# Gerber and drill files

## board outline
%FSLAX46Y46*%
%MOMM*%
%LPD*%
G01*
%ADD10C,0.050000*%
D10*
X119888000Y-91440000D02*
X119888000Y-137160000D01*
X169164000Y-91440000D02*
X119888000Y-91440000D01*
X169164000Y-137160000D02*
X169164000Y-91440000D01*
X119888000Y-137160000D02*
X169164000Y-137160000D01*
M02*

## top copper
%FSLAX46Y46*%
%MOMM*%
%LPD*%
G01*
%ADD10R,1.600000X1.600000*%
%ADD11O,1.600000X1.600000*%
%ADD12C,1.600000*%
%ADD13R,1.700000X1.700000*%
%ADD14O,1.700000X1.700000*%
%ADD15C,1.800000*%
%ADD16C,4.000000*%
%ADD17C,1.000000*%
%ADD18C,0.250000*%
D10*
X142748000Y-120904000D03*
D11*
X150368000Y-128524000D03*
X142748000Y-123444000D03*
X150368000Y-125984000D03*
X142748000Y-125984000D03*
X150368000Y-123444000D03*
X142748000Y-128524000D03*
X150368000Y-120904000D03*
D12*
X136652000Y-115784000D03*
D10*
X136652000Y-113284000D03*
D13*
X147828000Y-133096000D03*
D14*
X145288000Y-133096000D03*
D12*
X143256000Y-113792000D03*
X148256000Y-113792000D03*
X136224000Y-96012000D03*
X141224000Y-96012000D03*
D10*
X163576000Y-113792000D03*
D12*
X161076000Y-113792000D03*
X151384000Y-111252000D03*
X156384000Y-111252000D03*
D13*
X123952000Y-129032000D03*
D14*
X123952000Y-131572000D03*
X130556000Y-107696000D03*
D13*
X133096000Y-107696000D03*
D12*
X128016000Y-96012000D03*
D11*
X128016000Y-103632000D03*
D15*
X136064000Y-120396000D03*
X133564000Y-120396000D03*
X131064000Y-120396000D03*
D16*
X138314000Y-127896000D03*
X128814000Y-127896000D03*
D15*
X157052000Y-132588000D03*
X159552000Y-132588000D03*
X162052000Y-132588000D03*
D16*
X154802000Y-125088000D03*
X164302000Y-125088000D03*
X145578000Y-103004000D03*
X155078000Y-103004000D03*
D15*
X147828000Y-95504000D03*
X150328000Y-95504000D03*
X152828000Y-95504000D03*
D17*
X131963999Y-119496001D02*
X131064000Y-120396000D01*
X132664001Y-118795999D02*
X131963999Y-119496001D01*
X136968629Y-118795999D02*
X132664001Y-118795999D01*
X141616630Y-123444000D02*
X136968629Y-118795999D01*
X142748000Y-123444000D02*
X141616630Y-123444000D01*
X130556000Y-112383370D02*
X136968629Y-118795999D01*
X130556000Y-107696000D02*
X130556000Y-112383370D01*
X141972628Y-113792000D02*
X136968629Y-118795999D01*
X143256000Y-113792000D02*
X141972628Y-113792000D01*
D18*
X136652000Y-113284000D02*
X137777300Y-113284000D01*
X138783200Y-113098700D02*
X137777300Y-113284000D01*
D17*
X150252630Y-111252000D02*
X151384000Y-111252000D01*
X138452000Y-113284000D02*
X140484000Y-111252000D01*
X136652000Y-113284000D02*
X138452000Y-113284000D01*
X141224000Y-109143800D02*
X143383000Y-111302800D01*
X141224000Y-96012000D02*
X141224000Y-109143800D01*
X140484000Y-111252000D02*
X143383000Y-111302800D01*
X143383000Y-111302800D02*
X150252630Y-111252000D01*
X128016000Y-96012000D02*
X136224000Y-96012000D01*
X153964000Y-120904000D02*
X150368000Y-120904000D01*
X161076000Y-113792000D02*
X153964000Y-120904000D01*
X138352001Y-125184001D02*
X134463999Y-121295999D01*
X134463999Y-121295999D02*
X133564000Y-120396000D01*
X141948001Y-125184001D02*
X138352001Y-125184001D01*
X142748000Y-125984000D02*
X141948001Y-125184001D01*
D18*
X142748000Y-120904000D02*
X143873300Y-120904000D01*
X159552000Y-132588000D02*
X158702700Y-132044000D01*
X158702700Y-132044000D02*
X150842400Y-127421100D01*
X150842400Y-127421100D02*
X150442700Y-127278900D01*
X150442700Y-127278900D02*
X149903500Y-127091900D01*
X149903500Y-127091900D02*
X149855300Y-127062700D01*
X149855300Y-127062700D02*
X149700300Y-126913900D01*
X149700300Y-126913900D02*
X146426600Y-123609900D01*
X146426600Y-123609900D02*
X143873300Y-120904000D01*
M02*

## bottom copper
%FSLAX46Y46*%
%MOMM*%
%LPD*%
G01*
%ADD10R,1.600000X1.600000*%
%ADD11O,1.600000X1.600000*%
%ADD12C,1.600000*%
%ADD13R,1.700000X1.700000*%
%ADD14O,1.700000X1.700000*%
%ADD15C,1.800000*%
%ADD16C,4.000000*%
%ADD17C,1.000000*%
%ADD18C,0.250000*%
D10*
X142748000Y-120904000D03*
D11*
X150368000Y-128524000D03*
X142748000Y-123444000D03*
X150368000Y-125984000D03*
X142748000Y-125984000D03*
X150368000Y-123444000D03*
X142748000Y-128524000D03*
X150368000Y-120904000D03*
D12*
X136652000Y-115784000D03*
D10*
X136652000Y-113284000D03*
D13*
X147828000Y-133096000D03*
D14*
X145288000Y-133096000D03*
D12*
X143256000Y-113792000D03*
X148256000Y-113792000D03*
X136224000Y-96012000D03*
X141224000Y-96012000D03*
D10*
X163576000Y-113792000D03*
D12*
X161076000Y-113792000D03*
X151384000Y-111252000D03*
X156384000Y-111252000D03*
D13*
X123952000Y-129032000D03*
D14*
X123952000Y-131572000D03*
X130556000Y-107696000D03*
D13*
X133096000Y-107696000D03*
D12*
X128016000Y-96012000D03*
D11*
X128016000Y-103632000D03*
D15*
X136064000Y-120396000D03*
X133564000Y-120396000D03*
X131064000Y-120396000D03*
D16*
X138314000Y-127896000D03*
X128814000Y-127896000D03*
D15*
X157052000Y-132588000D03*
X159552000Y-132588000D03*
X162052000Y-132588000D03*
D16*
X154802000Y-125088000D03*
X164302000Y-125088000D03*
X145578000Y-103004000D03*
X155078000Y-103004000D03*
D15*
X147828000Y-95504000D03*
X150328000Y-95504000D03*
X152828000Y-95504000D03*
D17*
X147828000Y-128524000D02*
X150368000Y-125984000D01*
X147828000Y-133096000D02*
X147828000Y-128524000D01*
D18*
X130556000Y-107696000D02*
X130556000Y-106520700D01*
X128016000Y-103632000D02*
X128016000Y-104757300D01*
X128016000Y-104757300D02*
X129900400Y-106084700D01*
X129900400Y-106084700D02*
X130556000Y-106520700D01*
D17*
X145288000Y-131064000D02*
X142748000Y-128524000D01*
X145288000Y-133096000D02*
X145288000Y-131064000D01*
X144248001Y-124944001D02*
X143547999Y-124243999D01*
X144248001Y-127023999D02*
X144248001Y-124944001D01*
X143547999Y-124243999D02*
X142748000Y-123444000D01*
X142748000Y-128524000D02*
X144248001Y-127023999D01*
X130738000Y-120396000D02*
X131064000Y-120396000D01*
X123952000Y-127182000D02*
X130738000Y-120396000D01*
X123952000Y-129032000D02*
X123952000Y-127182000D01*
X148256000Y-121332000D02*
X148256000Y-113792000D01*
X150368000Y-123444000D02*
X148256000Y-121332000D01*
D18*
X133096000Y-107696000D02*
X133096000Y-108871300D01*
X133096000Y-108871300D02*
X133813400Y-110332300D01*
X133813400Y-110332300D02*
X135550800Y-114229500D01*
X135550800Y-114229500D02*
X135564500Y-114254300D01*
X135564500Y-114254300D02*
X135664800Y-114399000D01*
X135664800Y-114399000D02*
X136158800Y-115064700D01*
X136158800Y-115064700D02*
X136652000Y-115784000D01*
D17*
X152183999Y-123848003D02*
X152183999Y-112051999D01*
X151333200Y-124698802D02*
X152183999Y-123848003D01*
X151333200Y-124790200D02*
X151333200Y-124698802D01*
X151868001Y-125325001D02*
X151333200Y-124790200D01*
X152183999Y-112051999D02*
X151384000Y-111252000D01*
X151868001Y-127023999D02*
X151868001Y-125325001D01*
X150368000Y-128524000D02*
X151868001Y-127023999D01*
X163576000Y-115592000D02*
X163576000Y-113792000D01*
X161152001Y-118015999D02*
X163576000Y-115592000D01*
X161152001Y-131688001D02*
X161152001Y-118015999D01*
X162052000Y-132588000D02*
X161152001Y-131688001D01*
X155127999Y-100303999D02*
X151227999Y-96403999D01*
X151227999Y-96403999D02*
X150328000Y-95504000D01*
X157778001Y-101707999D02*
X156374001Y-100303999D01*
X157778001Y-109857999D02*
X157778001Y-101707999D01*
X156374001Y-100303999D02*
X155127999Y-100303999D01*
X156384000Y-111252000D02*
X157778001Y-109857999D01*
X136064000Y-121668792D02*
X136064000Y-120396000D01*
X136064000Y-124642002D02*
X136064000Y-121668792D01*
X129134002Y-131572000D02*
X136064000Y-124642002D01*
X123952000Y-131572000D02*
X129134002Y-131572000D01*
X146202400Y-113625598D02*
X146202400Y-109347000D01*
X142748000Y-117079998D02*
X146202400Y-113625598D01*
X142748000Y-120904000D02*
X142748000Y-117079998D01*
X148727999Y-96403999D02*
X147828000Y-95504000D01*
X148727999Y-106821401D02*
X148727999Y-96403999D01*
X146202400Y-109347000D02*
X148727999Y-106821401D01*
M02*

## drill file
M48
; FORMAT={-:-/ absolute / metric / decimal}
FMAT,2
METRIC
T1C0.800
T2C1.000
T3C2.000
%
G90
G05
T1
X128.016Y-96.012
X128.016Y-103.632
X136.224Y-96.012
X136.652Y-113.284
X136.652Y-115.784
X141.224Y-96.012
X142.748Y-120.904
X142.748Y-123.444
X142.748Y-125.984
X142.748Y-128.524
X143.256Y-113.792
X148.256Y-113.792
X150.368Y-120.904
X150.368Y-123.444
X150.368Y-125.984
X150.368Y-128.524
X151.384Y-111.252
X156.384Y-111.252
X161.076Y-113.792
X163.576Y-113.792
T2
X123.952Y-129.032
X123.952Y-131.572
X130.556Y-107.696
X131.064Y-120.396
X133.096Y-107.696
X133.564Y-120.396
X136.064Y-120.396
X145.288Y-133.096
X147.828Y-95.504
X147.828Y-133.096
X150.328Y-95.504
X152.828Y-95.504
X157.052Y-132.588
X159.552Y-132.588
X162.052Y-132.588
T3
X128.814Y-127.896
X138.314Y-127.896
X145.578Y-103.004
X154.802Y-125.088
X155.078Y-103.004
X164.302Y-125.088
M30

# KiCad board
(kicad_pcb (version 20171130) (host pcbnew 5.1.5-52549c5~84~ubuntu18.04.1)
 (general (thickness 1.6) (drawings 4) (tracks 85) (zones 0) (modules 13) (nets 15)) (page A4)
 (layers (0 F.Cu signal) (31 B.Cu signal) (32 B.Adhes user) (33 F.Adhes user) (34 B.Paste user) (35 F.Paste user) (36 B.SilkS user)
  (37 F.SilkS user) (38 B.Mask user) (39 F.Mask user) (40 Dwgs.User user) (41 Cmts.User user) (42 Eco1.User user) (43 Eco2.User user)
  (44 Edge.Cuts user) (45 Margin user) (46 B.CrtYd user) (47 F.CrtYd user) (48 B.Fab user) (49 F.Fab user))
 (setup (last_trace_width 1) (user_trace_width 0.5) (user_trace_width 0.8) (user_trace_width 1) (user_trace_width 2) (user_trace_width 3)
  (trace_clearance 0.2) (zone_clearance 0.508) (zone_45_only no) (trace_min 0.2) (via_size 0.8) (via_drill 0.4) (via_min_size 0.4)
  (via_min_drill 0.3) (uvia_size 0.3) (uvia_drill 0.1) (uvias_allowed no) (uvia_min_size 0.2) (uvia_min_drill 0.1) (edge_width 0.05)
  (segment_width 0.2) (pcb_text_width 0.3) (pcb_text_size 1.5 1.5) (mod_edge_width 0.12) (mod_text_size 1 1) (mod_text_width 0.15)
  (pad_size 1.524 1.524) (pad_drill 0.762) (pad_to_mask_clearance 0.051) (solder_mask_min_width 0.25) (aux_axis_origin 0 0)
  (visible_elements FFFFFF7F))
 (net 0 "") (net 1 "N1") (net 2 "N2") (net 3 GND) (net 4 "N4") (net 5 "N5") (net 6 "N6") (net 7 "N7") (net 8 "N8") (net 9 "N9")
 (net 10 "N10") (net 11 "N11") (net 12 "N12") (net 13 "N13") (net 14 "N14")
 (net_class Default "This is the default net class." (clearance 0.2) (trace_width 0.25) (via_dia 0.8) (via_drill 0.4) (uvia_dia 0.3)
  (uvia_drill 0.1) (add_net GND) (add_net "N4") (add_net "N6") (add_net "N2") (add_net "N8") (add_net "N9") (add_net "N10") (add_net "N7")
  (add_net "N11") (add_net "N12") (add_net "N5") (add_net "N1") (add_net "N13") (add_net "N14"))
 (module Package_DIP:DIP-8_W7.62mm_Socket (layer F.Cu) (at 142.748 120.904)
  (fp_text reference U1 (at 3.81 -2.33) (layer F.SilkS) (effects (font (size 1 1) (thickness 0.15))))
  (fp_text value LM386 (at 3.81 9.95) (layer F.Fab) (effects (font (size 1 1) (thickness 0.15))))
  (pad 1 thru_hole rect (at 0 0) (size 1.6 1.6) (drill 0.8) (layers *.Cu *.Mask) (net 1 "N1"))
  (pad 5 thru_hole oval (at 7.62 7.62) (size 1.6 1.6) (drill 0.8) (layers *.Cu *.Mask) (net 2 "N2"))
  (pad 2 thru_hole oval (at 0 2.54) (size 1.6 1.6) (drill 0.8) (layers *.Cu *.Mask) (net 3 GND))
  (pad 6 thru_hole oval (at 7.62 5.08) (size 1.6 1.6) (drill 0.8) (layers *.Cu *.Mask) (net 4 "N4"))
  (pad 3 thru_hole oval (at 0 5.08) (size 1.6 1.6) (drill 0.8) (layers *.Cu *.Mask) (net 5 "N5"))
  (pad 7 thru_hole oval (at 7.62 2.54) (size 1.6 1.6) (drill 0.8) (layers *.Cu *.Mask) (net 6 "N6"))
  (pad 4 thru_hole oval (at 0 7.62) (size 1.6 1.6) (drill 0.8) (layers *.Cu *.Mask) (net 3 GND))
  (pad 8 thru_hole oval (at 7.62 0) (size 1.6 1.6) (drill 0.8) (layers *.Cu *.Mask) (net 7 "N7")))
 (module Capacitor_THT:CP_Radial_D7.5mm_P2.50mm (layer F.Cu) (at 136.652 113.284 270)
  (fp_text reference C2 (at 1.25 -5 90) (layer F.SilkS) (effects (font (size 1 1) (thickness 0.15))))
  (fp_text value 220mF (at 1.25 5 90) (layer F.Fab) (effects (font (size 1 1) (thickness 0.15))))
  (pad 2 thru_hole circle (at 2.5 0 270) (size 1.6 1.6) (drill 0.8) (layers *.Cu *.Mask) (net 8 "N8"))
  (pad 1 thru_hole rect (at 0 0 270) (size 1.6 1.6) (drill 0.8) (layers *.Cu *.Mask) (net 2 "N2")))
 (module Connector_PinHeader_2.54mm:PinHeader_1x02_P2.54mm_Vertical (layer F.Cu) (at 147.828 133.096 270)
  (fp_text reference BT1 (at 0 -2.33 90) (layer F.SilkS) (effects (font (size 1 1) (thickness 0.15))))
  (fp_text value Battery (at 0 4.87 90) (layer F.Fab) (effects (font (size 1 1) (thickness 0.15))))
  (pad 1 thru_hole rect (at 0 0 270) (size 1.7 1.7) (drill 1) (layers *.Cu *.Mask) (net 4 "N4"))
  (pad 2 thru_hole oval (at 0 2.54 270) (size 1.7 1.7) (drill 1) (layers *.Cu *.Mask) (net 3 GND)))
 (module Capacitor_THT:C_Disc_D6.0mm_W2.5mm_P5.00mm (layer F.Cu) (at 143.256 113.792)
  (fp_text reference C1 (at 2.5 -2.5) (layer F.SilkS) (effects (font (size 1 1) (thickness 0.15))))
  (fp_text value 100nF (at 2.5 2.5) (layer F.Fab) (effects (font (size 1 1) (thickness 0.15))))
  (pad 1 thru_hole circle (at 0 0) (size 1.6 1.6) (drill 0.8) (layers *.Cu *.Mask) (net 3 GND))
  (pad 2 thru_hole circle (at 5 0) (size 1.6 1.6) (drill 0.8) (layers *.Cu *.Mask) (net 6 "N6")))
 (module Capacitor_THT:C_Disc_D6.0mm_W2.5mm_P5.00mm (layer F.Cu) (at 141.224 96.012 180)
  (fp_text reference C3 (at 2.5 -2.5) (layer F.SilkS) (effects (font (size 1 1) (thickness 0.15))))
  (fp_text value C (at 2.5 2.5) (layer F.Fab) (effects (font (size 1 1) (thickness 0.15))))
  (pad 2 thru_hole circle (at 5 0 180) (size 1.6 1.6) (drill 0.8) (layers *.Cu *.Mask) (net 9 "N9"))
  (pad 1 thru_hole circle (at 0 0 180) (size 1.6 1.6) (drill 0.8) (layers *.Cu *.Mask) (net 2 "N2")))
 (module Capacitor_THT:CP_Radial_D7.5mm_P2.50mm (layer F.Cu) (at 163.576 113.792 180)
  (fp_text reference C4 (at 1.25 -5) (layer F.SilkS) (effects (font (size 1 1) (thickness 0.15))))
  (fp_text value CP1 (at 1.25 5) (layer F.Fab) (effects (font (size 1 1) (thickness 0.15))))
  (pad 1 thru_hole rect (at 0 0 180) (size 1.6 1.6) (drill 0.8) (layers *.Cu *.Mask) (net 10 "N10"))
  (pad 2 thru_hole circle (at 2.5 0 180) (size 1.6 1.6) (drill 0.8) (layers *.Cu *.Mask) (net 7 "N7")))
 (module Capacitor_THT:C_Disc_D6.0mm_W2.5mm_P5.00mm (layer F.Cu) (at 151.384 111.252)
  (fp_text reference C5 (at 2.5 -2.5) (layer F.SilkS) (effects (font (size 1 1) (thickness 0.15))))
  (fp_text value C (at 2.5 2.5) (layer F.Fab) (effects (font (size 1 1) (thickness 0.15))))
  (pad 1 thru_hole circle (at 0 0) (size 1.6 1.6) (drill 0.8) (layers *.Cu *.Mask) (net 2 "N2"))
  (pad 2 thru_hole circle (at 5 0) (size 1.6 1.6) (drill 0.8) (layers *.Cu *.Mask) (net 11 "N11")))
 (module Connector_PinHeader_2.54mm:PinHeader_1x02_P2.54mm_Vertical (layer F.Cu) (at 123.952 129.032)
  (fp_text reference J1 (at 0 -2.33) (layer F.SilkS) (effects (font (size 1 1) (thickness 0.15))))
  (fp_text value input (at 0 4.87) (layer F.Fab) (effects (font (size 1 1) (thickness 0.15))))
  (pad 1 thru_hole rect (at 0 0) (size 1.7 1.7) (drill 1) (layers *.Cu *.Mask) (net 3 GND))
  (pad 2 thru_hole oval (at 0 2.54) (size 1.7 1.7) (drill 1) (layers *.Cu *.Mask) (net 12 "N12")))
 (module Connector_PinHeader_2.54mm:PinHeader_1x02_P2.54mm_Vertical (layer F.Cu) (at 133.096 107.696 270)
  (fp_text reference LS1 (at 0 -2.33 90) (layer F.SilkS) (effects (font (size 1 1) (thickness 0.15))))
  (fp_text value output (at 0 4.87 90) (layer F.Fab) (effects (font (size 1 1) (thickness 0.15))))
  (pad 2 thru_hole oval (at 0 2.54 270) (size 1.7 1.7) (drill 1) (layers *.Cu *.Mask) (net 3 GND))
  (pad 1 thru_hole rect (at 0 0 270) (size 1.7 1.7) (drill 1) (layers *.Cu *.Mask) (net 8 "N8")))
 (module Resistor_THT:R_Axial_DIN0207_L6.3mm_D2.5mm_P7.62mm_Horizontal (layer F.Cu) (at 128.016 96.012 270)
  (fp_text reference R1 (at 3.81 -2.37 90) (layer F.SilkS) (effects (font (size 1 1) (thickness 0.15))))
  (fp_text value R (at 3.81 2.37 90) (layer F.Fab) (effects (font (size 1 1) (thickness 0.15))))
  (pad 1 thru_hole circle (at 0 0 270) (size 1.6 1.6) (drill 0.8) (layers *.Cu *.Mask) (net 9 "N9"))
  (pad 2 thru_hole oval (at 7.62 0 270) (size 1.6 1.6) (drill 0.8) (layers *.Cu *.Mask) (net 3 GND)))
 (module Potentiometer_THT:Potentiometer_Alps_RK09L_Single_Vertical (layer F.Cu) (at 131.064 120.396 270)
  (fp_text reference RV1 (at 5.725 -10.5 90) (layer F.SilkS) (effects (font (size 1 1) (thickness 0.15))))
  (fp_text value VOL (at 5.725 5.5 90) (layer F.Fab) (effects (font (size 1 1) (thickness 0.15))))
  (pad 3 thru_hole circle (at 0 -5 270) (size 1.8 1.8) (drill 1) (layers *.Cu *.Mask) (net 12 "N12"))
  (pad 2 thru_hole circle (at 0 -2.5 270) (size 1.8 1.8) (drill 1) (layers *.Cu *.Mask) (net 5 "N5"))
  (pad 1 thru_hole circle (at 0 0 270) (size 1.8 1.8) (drill 1) (layers *.Cu *.Mask) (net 3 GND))
  (pad "" np_thru_hole circle (at 7.5 -7.25 270) (size 4 4) (drill 2) (layers *.Cu *.Mask))
  (pad "" np_thru_hole circle (at 7.5 2.25 270) (size 4 4) (drill 2) (layers *.Cu *.Mask)))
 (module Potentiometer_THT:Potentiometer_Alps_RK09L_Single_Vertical (layer F.Cu) (at 162.052 132.588 90)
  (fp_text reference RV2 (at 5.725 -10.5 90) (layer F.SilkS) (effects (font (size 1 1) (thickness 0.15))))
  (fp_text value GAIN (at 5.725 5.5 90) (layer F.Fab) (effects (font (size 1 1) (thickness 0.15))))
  (pad 3 thru_hole circle (at 0 -5 90) (size 1.8 1.8) (drill 1) (layers *.Cu *.Mask) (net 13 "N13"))
  (pad 2 thru_hole circle (at 0 -2.5 90) (size 1.8 1.8) (drill 1) (layers *.Cu *.Mask) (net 1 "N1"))
  (pad 1 thru_hole circle (at 0 0 90) (size 1.8 1.8) (drill 1) (layers *.Cu *.Mask) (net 10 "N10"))
  (pad "" np_thru_hole circle (at 7.5 -7.25 90) (size 4 4) (drill 2) (layers *.Cu *.Mask))
  (pad "" np_thru_hole circle (at 7.5 2.25 90) (size 4 4) (drill 2) (layers *.Cu *.Mask)))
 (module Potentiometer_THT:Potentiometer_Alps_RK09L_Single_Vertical (layer F.Cu) (at 147.828 95.504 270)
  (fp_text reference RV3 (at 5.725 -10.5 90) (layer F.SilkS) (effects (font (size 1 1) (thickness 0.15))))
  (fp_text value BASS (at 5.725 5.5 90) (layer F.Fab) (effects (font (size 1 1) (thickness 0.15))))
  (pad "" np_thru_hole circle (at 7.5 2.25 270) (size 4 4) (drill 2) (layers *.Cu *.Mask))
  (pad "" np_thru_hole circle (at 7.5 -7.25 270) (size 4 4) (drill 2) (layers *.Cu *.Mask))
  (pad 1 thru_hole circle (at 0 0 270) (size 1.8 1.8) (drill 1) (layers *.Cu *.Mask) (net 1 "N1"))
  (pad 2 thru_hole circle (at 0 -2.5 270) (size 1.8 1.8) (drill 1) (layers *.Cu *.Mask) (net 11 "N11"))
  (pad 3 thru_hole circle (at 0 -5 270) (size 1.8 1.8) (drill 1) (layers *.Cu *.Mask) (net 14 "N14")))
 (gr_line (start 119.888 91.44) (end 119.888 137.16) (layer Edge.Cuts) (width 0.05))
 (gr_line (start 169.164 91.44) (end 119.888 91.44) (layer Edge.Cuts) (width 0.05))
 (gr_line (start 169.164 137.16) (end 169.164 91.44) (layer Edge.Cuts) (width 0.05))
 (gr_line (start 119.888 137.16) (end 169.164 137.16) (layer Edge.Cuts) (width 0.05))
 (segment (start 147.828 128.524) (end 150.368 125.984) (width 1) (layer B.Cu) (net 4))
 (segment (start 147.828 133.096) (end 147.828 128.524) (width 1) (layer B.Cu) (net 4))
 (segment (start 130.556 107.696) (end 130.556 106.5207) (width 0.25) (layer B.Cu) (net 3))
 (segment (start 128.016 103.632) (end 128.016 104.7573) (width 0.25) (layer B.Cu) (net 3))
 (segment (start 128.016 104.7573) (end 129.9004 106.0847) (width 0.25) (layer B.Cu) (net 3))
 (segment (start 129.9004 106.0847) (end 130.556 106.5207) (width 0.25) (layer B.Cu) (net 3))
 (segment (start 131.963999 119.496001) (end 131.064 120.396) (width 1) (layer F.Cu) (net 3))
 (segment (start 132.664001 118.795999) (end 131.963999 119.496001) (width 1) (layer F.Cu) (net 3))
 (segment (start 136.968629 118.795999) (end 132.664001 118.795999) (width 1) (layer F.Cu) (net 3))
 (segment (start 141.61663 123.444) (end 136.968629 118.795999) (width 1) (layer F.Cu) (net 3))
 (segment (start 142.748 123.444) (end 141.61663 123.444) (width 1) (layer F.Cu) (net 3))
 (segment (start 130.556 112.38337) (end 136.968629 118.795999) (width 1) (layer F.Cu) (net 3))
 (segment (start 130.556 107.696) (end 130.556 112.38337) (width 1) (layer F.Cu) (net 3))
 (segment (start 141.972628 113.792) (end 136.968629 118.795999) (width 1) (layer F.Cu) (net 3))
 (segment (start 143.256 113.792) (end 141.972628 113.792) (width 1) (layer F.Cu) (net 3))
 (segment (start 145.288 131.064) (end 142.748 128.524) (width 1) (layer B.Cu) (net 3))
 (segment (start 145.288 133.096) (end 145.288 131.064) (width 1) (layer B.Cu) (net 3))
 (segment (start 144.248001 124.944001) (end 143.547999 124.243999) (width 1) (layer B.Cu) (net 3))
 (segment (start 144.248001 127.023999) (end 144.248001 124.944001) (width 1) (layer B.Cu) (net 3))
 (segment (start 143.547999 124.243999) (end 142.748 123.444) (width 1) (layer B.Cu) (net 3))
 (segment (start 142.748 128.524) (end 144.248001 127.023999) (width 1) (layer B.Cu) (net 3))
 (segment (start 130.738 120.396) (end 131.064 120.396) (width 1) (layer B.Cu) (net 3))
 (segment (start 123.952 127.182) (end 130.738 120.396) (width 1) (layer B.Cu) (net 3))
 (segment (start 123.952 129.032) (end 123.952 127.182) (width 1) (layer B.Cu) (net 3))
 (segment (start 148.256 121.332) (end 148.256 113.792) (width 1) (layer B.Cu) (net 6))
 (segment (start 150.368 123.444) (end 148.256 121.332) (width 1) (layer B.Cu) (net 6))
 (segment (start 133.096 107.696) (end 133.096 108.8713) (width 0.25) (layer B.Cu) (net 8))
 (segment (start 133.096 108.8713) (end 133.8134 110.3323) (width 0.25) (layer B.Cu) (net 8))
 (segment (start 133.8134 110.3323) (end 135.5508 114.2295) (width 0.25) (layer B.Cu) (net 8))
 (segment (start 135.5508 114.2295) (end 135.5645 114.2543) (width 0.25) (layer B.Cu) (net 8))
 (segment (start 135.5645 114.2543) (end 135.6648 114.399) (width 0.25) (layer B.Cu) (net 8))
 (segment (start 135.6648 114.399) (end 136.1588 115.0647) (width 0.25) (layer B.Cu) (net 8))
 (segment (start 136.1588 115.0647) (end 136.652 115.784) (width 0.25) (layer B.Cu) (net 8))
 (segment (start 136.652 113.284) (end 137.7773 113.284) (width 0.25) (layer F.Cu) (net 2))
 (segment (start 138.7832 113.0987) (end 137.7773 113.284) (width 0.25) (layer F.Cu) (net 2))
 (segment (start 150.25263 111.252) (end 151.384 111.252) (width 1) (layer F.Cu) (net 2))
 (segment (start 138.452 113.284) (end 140.484 111.252) (width 1) (layer F.Cu) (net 2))
 (segment (start 136.652 113.284) (end 138.452 113.284) (width 1) (layer F.Cu) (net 2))
 (segment (start 141.224 109.1438) (end 143.383 111.3028) (width 1) (layer F.Cu) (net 2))
 (segment (start 141.224 96.012) (end 141.224 109.1438) (width 1) (layer F.Cu) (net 2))
 (segment (start 140.484 111.252) (end 143.383 111.3028) (width 1) (layer F.Cu) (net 2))
 (segment (start 143.383 111.3028) (end 150.25263 111.252) (width 1) (layer F.Cu) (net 2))
 (segment (start 152.183999 123.848003) (end 152.183999 112.051999) (width 1) (layer B.Cu) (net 2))
 (segment (start 151.3332 124.698802) (end 152.183999 123.848003) (width 1) (layer B.Cu) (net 2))
 (segment (start 151.3332 124.7902) (end 151.3332 124.698802) (width 1) (layer B.Cu) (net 2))
 (segment (start 151.868001 125.325001) (end 151.3332 124.7902) (width 1) (layer B.Cu) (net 2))
 (segment (start 152.183999 112.051999) (end 151.384 111.252) (width 1) (layer B.Cu) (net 2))
 (segment (start 151.868001 127.023999) (end 151.868001 125.325001) (width 1) (layer B.Cu) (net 2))
 (segment (start 150.368 128.524) (end 151.868001 127.023999) (width 1) (layer B.Cu) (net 2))
 (segment (start 128.016 96.012) (end 136.224 96.012) (width 1) (layer F.Cu) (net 9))
 (segment (start 163.576 115.592) (end 163.576 113.792) (width 1) (layer B.Cu) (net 10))
 (segment (start 161.152001 118.015999) (end 163.576 115.592) (width 1) (layer B.Cu) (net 10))
 (segment (start 161.152001 131.688001) (end 161.152001 118.015999) (width 1) (layer B.Cu) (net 10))
 (segment (start 162.052 132.588) (end 161.152001 131.688001) (width 1) (layer B.Cu) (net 10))
 (segment (start 153.964 120.904) (end 150.368 120.904) (width 1) (layer F.Cu) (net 7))
 (segment (start 161.076 113.792) (end 153.964 120.904) (width 1) (layer F.Cu) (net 7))
 (segment (start 155.127999 100.303999) (end 151.227999 96.403999) (width 1) (layer B.Cu) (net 11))
 (segment (start 151.227999 96.403999) (end 150.328 95.504) (width 1) (layer B.Cu) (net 11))
 (segment (start 157.778001 101.707999) (end 156.374001 100.303999) (width 1) (layer B.Cu) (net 11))
 (segment (start 157.778001 109.857999) (end 157.778001 101.707999) (width 1) (layer B.Cu) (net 11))
 (segment (start 156.374001 100.303999) (end 155.127999 100.303999) (width 1) (layer B.Cu) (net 11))
 (segment (start 156.384 111.252) (end 157.778001 109.857999) (width 1) (layer B.Cu) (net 11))
 (segment (start 136.064 121.668792) (end 136.064 120.396) (width 1) (layer B.Cu) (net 12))
 (segment (start 136.064 124.642002) (end 136.064 121.668792) (width 1) (layer B.Cu) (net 12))
 (segment (start 129.134002 131.572) (end 136.064 124.642002) (width 1) (layer B.Cu) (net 12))
 (segment (start 123.952 131.572) (end 129.134002 131.572) (width 1) (layer B.Cu) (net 12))
 (segment (start 138.352001 125.184001) (end 134.463999 121.295999) (width 1) (layer F.Cu) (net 5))
 (segment (start 134.463999 121.295999) (end 133.564 120.396) (width 1) (layer F.Cu) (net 5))
 (segment (start 141.948001 125.184001) (end 138.352001 125.184001) (width 1) (layer F.Cu) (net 5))
 (segment (start 142.748 125.984) (end 141.948001 125.184001) (width 1) (layer F.Cu) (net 5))
 (segment (start 142.748 120.904) (end 143.8733 120.904) (width 0.25) (layer F.Cu) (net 1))
 (segment (start 159.552 132.588) (end 158.7027 132.044) (width 0.25) (layer F.Cu) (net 1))
 (segment (start 158.7027 132.044) (end 150.8424 127.4211) (width 0.25) (layer F.Cu) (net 1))
 (segment (start 150.8424 127.4211) (end 150.4427 127.2789) (width 0.25) (layer F.Cu) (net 1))
 (segment (start 150.4427 127.2789) (end 149.9035 127.0919) (width 0.25) (layer F.Cu) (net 1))
 (segment (start 149.9035 127.0919) (end 149.8553 127.0627) (width 0.25) (layer F.Cu) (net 1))
 (segment (start 149.8553 127.0627) (end 149.7003 126.9139) (width 0.25) (layer F.Cu) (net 1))
 (segment (start 149.7003 126.9139) (end 146.4266 123.6099) (width 0.25) (layer F.Cu) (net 1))
 (segment (start 146.4266 123.6099) (end 143.8733 120.904) (width 0.25) (layer F.Cu) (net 1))
 (segment (start 146.2024 113.625598) (end 146.2024 109.347) (width 1) (layer B.Cu) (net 1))
 (segment (start 142.748 117.079998) (end 146.2024 113.625598) (width 1) (layer B.Cu) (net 1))
 (segment (start 142.748 120.904) (end 142.748 117.079998) (width 1) (layer B.Cu) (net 1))
 (segment (start 148.727999 96.403999) (end 147.828 95.504) (width 1) (layer B.Cu) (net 1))
 (segment (start 148.727999 106.821401) (end 148.727999 96.403999) (width 1) (layer B.Cu) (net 1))
 (segment (start 146.2024 109.347) (end 148.727999 106.821401) (width 1) (layer B.Cu) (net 1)))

